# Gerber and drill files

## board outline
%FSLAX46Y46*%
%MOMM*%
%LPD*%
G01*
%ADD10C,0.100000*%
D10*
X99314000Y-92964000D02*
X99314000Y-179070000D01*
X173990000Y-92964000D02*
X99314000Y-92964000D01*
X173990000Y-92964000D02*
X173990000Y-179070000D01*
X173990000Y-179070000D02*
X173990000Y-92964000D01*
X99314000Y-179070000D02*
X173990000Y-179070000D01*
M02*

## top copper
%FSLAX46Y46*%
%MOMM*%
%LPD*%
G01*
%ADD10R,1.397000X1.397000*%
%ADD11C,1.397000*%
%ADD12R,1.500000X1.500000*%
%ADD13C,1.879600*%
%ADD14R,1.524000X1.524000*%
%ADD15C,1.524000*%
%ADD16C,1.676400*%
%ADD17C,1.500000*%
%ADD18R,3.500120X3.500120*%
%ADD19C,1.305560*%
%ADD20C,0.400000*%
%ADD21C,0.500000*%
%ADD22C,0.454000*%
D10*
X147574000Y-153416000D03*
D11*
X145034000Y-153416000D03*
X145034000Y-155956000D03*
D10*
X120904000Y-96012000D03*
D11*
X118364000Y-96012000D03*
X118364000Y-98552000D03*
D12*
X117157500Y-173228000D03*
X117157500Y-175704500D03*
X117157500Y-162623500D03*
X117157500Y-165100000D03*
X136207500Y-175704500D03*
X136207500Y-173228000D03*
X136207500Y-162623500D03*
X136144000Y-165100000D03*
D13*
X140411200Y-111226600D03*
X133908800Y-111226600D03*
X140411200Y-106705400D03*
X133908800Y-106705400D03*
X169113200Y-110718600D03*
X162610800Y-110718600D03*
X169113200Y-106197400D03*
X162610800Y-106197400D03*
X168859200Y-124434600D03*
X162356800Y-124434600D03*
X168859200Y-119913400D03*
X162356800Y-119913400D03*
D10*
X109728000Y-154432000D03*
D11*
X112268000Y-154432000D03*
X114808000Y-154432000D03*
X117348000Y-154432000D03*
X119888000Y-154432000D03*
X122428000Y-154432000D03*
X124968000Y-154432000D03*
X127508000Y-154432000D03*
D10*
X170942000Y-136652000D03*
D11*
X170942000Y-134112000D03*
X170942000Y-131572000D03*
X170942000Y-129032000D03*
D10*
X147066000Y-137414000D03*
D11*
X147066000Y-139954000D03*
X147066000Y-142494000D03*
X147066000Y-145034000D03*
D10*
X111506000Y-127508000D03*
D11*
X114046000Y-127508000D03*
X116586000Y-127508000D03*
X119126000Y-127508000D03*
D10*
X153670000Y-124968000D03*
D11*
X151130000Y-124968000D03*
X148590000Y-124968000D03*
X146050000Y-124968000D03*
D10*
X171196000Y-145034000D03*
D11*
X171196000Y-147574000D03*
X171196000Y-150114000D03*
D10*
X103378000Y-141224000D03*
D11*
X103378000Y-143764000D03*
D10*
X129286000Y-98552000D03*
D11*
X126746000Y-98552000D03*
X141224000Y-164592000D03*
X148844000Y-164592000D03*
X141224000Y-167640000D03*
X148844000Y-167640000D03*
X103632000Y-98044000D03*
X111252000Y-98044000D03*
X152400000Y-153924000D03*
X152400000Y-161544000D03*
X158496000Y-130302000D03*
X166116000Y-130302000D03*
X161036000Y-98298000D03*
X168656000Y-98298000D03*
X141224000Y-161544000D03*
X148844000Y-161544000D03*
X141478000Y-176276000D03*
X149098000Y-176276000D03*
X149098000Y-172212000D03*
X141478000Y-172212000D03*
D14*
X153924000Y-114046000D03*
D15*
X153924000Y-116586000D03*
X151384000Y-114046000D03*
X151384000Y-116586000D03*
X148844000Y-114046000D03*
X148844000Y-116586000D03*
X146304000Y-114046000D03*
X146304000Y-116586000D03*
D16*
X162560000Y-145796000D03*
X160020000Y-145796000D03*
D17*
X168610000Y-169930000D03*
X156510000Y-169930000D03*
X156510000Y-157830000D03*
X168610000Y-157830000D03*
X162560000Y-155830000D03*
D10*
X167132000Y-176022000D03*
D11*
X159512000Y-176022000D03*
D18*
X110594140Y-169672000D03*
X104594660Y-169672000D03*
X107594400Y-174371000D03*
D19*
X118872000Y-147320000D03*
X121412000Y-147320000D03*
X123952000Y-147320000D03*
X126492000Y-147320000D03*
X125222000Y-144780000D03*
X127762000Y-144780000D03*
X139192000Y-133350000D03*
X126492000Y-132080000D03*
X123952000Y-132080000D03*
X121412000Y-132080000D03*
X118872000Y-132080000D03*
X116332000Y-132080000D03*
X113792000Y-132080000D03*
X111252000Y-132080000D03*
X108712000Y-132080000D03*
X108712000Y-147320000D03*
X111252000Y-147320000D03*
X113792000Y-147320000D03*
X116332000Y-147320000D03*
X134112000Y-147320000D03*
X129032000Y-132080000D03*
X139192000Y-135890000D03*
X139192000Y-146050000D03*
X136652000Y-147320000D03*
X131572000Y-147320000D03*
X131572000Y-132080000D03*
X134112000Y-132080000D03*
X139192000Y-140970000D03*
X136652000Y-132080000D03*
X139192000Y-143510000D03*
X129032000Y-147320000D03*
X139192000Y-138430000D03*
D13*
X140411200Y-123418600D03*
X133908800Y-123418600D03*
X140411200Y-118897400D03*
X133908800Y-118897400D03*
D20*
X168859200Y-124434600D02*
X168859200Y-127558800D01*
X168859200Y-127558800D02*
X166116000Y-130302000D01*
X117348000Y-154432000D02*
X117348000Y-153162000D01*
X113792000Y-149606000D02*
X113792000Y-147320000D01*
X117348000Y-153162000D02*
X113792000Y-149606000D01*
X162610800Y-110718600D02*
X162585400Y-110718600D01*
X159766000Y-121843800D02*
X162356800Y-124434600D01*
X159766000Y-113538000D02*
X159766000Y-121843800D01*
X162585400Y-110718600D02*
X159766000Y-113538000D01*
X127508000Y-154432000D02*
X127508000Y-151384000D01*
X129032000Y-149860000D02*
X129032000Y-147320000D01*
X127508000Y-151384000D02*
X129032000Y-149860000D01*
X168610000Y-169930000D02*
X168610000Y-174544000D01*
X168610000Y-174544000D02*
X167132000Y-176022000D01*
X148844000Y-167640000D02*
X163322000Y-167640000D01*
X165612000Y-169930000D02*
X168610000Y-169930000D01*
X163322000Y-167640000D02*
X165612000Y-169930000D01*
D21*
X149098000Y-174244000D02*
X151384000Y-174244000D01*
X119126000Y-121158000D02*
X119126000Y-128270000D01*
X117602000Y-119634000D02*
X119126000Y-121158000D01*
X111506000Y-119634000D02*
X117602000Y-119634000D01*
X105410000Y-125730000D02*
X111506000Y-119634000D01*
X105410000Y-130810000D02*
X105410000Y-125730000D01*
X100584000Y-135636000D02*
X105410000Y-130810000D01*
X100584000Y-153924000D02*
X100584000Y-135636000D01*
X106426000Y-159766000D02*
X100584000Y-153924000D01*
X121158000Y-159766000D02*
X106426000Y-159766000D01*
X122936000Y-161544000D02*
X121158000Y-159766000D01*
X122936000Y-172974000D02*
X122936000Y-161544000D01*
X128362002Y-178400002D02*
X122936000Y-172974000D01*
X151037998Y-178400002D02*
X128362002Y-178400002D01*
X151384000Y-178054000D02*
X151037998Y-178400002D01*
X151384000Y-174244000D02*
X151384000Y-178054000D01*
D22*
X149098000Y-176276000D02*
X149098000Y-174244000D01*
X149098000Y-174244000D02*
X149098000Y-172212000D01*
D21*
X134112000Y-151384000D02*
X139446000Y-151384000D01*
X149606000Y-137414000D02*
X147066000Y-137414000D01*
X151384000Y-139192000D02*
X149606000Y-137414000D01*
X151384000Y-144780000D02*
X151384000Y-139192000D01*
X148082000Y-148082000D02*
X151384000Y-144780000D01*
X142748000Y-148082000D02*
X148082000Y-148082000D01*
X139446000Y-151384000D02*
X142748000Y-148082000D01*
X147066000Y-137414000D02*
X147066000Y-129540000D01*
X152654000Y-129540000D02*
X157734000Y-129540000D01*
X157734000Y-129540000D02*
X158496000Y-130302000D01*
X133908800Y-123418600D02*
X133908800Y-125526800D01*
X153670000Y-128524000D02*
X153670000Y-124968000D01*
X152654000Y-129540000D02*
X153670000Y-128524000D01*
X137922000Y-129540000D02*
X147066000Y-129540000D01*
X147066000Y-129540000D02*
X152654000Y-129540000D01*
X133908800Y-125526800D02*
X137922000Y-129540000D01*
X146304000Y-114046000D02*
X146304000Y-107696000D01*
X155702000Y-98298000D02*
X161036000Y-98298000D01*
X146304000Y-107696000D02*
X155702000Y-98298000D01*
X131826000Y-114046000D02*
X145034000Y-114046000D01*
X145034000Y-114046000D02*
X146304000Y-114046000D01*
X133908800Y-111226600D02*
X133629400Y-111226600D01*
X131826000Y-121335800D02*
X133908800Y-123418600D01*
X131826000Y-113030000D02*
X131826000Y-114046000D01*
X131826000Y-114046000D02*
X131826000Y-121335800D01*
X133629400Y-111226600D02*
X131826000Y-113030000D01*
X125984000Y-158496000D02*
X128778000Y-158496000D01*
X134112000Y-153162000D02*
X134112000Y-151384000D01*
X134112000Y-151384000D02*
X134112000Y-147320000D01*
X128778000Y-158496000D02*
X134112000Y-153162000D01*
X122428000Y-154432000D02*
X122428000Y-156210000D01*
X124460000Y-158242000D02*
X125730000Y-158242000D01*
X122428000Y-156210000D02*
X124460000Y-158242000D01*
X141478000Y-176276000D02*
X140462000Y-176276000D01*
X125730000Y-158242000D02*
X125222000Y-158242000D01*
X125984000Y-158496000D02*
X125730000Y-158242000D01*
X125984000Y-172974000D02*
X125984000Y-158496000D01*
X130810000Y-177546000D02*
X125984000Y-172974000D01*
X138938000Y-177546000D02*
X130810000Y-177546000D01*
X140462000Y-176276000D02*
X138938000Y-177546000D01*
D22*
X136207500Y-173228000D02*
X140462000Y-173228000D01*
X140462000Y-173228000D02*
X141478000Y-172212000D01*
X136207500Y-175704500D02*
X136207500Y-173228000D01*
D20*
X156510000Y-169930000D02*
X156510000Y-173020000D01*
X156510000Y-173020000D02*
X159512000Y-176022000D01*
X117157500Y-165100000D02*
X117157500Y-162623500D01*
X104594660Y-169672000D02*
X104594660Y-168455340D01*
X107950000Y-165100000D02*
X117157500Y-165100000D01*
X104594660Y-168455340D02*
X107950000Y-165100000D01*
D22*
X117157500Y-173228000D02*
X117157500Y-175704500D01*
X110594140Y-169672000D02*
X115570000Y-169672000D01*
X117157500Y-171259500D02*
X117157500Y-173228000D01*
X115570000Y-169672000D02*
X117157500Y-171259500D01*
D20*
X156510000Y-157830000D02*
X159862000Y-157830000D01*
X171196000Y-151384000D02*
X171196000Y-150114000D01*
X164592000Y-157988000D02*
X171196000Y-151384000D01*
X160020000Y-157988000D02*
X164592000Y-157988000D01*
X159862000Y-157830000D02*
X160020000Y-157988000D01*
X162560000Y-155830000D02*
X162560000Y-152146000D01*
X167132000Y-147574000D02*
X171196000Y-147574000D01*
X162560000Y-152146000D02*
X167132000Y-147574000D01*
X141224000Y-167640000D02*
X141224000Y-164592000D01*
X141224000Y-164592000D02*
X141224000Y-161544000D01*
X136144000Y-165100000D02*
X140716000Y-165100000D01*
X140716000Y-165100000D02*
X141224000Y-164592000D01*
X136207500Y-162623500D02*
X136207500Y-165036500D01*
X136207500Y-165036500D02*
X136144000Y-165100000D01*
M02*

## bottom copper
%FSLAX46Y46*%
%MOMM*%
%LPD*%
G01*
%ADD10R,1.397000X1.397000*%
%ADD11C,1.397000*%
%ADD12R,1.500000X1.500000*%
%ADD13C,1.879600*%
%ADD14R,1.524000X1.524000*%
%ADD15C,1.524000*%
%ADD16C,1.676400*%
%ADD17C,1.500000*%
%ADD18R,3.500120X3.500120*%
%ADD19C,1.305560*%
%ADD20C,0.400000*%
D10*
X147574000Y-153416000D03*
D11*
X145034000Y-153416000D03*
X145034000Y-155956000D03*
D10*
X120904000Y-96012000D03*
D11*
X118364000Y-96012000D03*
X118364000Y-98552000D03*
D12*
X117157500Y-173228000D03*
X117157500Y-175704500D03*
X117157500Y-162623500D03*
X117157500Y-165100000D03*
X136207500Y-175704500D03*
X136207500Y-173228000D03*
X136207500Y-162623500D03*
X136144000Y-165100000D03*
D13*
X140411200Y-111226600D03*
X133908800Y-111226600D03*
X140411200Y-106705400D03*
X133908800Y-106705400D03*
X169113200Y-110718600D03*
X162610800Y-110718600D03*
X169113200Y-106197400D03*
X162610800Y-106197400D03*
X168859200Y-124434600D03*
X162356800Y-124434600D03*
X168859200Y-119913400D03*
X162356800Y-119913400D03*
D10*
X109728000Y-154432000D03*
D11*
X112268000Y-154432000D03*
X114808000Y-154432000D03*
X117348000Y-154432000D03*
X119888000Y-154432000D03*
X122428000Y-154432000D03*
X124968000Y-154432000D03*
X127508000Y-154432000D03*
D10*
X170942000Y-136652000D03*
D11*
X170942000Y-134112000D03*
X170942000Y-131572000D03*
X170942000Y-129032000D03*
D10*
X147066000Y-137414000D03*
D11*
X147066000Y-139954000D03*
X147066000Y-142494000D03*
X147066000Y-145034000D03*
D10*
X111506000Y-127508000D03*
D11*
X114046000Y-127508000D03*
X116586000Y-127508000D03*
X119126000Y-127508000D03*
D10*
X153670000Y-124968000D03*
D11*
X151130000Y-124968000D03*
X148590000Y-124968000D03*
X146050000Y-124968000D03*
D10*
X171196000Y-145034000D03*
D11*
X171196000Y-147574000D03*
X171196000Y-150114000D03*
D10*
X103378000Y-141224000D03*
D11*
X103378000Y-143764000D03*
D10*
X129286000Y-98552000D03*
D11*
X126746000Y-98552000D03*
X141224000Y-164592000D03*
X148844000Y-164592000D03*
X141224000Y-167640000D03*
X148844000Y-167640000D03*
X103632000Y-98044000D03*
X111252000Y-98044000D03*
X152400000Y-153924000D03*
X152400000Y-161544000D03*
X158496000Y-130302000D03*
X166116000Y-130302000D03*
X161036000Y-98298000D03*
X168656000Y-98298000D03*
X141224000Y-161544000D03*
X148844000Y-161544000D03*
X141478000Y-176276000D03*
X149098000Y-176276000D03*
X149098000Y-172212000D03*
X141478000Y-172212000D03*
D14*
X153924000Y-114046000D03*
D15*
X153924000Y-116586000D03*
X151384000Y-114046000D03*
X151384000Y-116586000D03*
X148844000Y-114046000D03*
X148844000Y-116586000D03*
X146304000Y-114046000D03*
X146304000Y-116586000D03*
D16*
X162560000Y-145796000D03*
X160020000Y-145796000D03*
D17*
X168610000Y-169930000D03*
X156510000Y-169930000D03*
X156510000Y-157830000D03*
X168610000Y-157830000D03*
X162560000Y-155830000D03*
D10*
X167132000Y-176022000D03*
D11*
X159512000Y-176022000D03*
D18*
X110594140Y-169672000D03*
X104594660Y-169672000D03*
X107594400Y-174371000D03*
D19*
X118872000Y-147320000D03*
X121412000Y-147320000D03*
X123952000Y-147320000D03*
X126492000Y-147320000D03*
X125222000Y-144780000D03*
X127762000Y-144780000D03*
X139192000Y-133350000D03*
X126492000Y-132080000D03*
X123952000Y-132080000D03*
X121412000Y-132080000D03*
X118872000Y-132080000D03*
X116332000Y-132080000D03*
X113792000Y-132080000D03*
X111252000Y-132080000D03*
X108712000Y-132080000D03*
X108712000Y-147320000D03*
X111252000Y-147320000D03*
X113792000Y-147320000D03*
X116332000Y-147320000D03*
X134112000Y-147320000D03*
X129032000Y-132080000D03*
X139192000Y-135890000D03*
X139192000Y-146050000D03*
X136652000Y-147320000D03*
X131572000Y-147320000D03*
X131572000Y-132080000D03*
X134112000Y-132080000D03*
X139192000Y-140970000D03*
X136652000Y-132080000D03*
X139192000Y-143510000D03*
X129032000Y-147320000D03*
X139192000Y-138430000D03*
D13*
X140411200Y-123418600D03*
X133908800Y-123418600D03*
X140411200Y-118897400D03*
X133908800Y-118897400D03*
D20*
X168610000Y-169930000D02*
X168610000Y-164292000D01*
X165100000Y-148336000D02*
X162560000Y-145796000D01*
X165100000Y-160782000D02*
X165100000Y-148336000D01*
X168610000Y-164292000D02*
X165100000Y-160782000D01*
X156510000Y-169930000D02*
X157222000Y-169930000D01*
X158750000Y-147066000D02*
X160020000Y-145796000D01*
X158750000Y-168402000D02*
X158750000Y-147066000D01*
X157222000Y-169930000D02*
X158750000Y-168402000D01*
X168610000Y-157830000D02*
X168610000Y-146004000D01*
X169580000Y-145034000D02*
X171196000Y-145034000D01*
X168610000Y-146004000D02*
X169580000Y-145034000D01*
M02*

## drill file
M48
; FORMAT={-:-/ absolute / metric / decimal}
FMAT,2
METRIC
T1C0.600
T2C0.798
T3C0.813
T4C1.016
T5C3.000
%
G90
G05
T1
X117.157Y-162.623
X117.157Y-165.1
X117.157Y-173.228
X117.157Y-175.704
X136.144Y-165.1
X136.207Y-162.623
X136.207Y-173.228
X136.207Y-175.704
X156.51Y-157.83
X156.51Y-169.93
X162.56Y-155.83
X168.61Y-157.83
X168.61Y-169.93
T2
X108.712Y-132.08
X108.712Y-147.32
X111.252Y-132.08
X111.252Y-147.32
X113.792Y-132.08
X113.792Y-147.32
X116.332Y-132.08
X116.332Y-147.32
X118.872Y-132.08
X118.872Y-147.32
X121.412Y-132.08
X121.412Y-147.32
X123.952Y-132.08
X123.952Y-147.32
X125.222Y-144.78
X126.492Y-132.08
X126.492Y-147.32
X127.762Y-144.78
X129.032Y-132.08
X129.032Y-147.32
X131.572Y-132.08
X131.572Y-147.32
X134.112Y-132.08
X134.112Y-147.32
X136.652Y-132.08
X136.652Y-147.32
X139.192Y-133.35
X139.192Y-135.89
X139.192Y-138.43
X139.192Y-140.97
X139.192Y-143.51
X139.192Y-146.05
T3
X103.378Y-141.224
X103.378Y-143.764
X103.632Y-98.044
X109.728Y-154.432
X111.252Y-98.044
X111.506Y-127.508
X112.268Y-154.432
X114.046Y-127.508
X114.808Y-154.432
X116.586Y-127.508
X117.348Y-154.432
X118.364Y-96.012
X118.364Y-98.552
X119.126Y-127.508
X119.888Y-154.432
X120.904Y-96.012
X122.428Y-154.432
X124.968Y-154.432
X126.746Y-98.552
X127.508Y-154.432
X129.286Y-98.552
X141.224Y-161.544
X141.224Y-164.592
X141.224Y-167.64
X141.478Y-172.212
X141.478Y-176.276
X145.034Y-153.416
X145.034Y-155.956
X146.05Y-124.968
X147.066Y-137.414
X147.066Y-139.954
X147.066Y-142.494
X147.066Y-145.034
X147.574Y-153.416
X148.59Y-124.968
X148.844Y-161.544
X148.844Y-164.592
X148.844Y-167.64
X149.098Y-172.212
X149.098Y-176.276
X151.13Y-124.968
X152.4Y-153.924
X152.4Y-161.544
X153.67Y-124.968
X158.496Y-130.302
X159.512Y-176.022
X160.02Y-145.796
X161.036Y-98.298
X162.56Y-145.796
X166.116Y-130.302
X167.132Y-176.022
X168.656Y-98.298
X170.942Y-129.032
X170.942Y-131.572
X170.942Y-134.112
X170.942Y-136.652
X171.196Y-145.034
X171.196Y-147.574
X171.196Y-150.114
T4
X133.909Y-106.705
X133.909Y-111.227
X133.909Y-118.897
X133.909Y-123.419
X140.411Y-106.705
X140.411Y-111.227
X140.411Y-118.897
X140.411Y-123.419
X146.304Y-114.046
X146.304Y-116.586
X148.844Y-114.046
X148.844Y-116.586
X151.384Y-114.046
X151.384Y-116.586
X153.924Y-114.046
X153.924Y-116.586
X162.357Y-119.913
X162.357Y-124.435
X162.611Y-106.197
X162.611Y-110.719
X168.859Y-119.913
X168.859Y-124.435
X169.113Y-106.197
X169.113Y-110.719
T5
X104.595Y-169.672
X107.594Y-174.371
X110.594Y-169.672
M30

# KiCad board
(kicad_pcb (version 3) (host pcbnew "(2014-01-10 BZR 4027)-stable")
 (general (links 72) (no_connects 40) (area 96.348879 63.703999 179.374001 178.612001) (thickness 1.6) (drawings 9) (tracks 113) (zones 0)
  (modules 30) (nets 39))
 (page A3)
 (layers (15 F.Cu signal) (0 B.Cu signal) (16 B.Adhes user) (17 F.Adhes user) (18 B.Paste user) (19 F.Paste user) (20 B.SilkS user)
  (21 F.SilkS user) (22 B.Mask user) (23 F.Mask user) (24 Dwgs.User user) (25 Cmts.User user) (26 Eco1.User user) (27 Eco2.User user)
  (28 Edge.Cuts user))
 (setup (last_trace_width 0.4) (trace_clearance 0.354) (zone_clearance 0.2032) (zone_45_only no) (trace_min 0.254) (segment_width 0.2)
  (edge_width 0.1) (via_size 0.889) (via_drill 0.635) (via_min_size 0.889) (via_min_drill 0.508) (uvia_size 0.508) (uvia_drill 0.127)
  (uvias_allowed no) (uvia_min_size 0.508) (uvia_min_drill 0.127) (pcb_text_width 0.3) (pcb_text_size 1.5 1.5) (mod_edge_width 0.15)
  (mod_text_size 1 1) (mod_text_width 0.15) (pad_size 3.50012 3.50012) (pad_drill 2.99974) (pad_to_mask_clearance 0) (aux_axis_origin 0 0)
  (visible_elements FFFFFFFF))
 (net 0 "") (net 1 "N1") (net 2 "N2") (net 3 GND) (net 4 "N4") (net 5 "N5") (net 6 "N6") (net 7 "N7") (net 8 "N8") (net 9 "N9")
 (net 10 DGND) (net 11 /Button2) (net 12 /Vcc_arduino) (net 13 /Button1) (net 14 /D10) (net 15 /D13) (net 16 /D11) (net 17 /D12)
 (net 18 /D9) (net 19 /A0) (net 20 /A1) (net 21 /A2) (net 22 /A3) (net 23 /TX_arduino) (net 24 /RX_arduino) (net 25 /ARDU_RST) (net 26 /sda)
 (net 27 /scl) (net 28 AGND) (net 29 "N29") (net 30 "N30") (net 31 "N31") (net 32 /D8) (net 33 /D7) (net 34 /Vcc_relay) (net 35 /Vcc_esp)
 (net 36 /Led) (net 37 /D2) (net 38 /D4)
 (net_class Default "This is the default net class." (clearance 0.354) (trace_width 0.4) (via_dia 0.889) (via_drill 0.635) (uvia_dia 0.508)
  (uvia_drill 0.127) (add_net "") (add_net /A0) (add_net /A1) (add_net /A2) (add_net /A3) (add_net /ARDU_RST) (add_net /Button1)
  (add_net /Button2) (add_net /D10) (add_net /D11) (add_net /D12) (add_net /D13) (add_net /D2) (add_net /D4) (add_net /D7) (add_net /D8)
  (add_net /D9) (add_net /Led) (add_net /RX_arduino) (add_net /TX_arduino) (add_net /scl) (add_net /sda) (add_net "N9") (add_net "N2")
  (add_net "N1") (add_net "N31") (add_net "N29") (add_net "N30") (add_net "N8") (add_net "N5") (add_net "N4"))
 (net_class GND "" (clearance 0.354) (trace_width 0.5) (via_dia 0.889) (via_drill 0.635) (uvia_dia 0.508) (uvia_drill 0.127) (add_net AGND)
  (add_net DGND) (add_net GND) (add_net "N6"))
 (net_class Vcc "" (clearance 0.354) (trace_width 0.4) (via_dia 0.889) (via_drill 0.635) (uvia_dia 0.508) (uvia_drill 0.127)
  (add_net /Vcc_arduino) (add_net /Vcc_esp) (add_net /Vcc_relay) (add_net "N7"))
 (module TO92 (layer F.Cu) (at 146.304 154.686)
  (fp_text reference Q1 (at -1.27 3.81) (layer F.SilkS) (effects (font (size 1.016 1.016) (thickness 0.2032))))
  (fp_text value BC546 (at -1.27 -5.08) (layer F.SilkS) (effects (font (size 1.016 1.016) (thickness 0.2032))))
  (pad 1 thru_hole rect (at 1.27 -1.27) (size 1.397 1.397) (drill 0.8128) (layers *.Cu *.Mask F.SilkS) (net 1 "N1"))
  (pad 2 thru_hole circle (at -1.27 -1.27) (size 1.397 1.397) (drill 0.8128) (layers *.Cu *.Mask F.SilkS) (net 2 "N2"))
  (pad 3 thru_hole circle (at -1.27 1.27) (size 1.397 1.397) (drill 0.8128) (layers *.Cu *.Mask F.SilkS) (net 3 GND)))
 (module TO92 (layer F.Cu) (at 119.634 97.282)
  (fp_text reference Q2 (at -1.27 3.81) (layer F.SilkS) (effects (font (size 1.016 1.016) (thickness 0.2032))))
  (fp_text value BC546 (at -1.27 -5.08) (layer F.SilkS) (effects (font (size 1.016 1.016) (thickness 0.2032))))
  (pad 1 thru_hole rect (at 1.27 -1.27) (size 1.397 1.397) (drill 0.8128) (layers *.Cu *.Mask F.SilkS) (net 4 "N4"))
  (pad 2 thru_hole circle (at -1.27 -1.27) (size 1.397 1.397) (drill 0.8128) (layers *.Cu *.Mask F.SilkS) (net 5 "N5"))
  (pad 3 thru_hole circle (at -1.27 1.27) (size 1.397 1.397) (drill 0.8128) (layers *.Cu *.Mask F.SilkS) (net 3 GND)))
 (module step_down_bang (layer F.Cu) (at 126.492 169.164 90)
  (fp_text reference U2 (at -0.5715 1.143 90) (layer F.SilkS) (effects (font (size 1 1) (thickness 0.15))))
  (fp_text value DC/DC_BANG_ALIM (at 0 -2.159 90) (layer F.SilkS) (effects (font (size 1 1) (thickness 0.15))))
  (pad 3 thru_hole rect (at -4.064 -9.3345 90) (size 1.5 1.5) (drill 0.6) (layers *.Cu *.Mask F.SilkS) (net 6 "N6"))
  (pad 4 thru_hole rect (at -6.5405 -9.3345 90) (size 1.5 1.5) (drill 0.6) (layers *.Cu *.Mask F.SilkS) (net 6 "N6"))
  (pad 1 thru_hole rect (at 6.5405 -9.3345 90) (size 1.5 1.5) (drill 0.6) (layers *.Cu *.Mask F.SilkS) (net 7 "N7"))
  (pad 2 thru_hole rect (at 4.064 -9.3345 90) (size 1.5 1.5) (drill 0.6) (layers *.Cu *.Mask F.SilkS) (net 7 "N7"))
  (pad 8 thru_hole rect (at -6.5405 9.7155 90) (size 1.5 1.5) (drill 0.6) (layers *.Cu *.Mask F.SilkS) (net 3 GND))
  (pad 7 thru_hole rect (at -4.064 9.7155 90) (size 1.5 1.5) (drill 0.6) (layers *.Cu *.Mask F.SilkS) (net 3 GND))
  (pad 5 thru_hole rect (at 6.5405 9.7155 90) (size 1.5 1.5) (drill 0.6) (layers *.Cu *.Mask F.SilkS) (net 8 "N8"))
  (pad 6 thru_hole rect (at 4.064 9.652 90) (size 1.5 1.5) (drill 0.6) (layers *.Cu *.Mask F.SilkS) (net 8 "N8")))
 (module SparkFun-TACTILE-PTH (layer F.Cu) (at 137.16 108.966 180)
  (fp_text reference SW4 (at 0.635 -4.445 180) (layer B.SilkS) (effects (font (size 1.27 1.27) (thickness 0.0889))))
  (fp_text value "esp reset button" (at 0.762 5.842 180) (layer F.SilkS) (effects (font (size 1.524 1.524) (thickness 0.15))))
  (pad 1 thru_hole circle (at -3.2512 -2.2606 180) (size 1.8796 1.8796) (drill 1.016) (layers *.Cu F.Paste F.SilkS F.Mask) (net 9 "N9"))
  (pad 2 thru_hole circle (at 3.2512 -2.2606 180) (size 1.8796 1.8796) (drill 1.016) (layers *.Cu F.Paste F.SilkS F.Mask) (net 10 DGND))
  (pad 3 thru_hole circle (at -3.2512 2.2606 180) (size 1.8796 1.8796) (drill 1.016) (layers *.Cu F.Paste F.SilkS F.Mask))
  (pad 4 thru_hole circle (at 3.2512 2.2606 180) (size 1.8796 1.8796) (drill 1.016) (layers *.Cu F.Paste F.SilkS F.Mask)))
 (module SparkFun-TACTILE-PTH (layer F.Cu) (at 165.862 108.458 180)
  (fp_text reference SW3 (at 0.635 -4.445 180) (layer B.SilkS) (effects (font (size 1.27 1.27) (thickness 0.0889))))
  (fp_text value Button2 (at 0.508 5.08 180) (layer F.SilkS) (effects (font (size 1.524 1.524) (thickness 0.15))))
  (pad 1 thru_hole circle (at -3.2512 -2.2606 180) (size 1.8796 1.8796) (drill 1.016) (layers *.Cu F.Paste F.SilkS F.Mask) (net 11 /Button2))
  (pad 2 thru_hole circle (at 3.2512 -2.2606 180) (size 1.8796 1.8796) (drill 1.016) (layers *.Cu F.Paste F.SilkS F.Mask)
   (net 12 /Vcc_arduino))
  (pad 3 thru_hole circle (at -3.2512 2.2606 180) (size 1.8796 1.8796) (drill 1.016) (layers *.Cu F.Paste F.SilkS F.Mask))
  (pad 4 thru_hole circle (at 3.2512 2.2606 180) (size 1.8796 1.8796) (drill 1.016) (layers *.Cu F.Paste F.SilkS F.Mask)))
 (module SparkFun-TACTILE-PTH (layer F.Cu) (at 165.608 122.174 180)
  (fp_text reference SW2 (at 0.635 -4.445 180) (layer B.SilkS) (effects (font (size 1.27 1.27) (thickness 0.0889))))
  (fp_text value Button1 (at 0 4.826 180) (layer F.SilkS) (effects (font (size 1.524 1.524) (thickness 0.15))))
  (pad 1 thru_hole circle (at -3.2512 -2.2606 180) (size 1.8796 1.8796) (drill 1.016) (layers *.Cu F.Paste F.SilkS F.Mask) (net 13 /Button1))
  (pad 2 thru_hole circle (at 3.2512 -2.2606 180) (size 1.8796 1.8796) (drill 1.016) (layers *.Cu F.Paste F.SilkS F.Mask)
   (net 12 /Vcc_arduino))
  (pad 3 thru_hole circle (at -3.2512 2.2606 180) (size 1.8796 1.8796) (drill 1.016) (layers *.Cu F.Paste F.SilkS F.Mask))
  (pad 4 thru_hole circle (at 3.2512 2.2606 180) (size 1.8796 1.8796) (drill 1.016) (layers *.Cu F.Paste F.SilkS F.Mask)))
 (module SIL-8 (layer F.Cu) (at 118.618 154.432)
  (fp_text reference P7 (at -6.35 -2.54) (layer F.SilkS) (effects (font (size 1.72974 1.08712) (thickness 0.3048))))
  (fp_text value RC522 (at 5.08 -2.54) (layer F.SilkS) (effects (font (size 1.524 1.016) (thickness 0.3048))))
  (pad 1 thru_hole rect (at -8.89 0) (size 1.397 1.397) (drill 0.8128) (layers *.Cu *.Mask F.SilkS) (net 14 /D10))
  (pad 2 thru_hole circle (at -6.35 0) (size 1.397 1.397) (drill 0.8128) (layers *.Cu *.Mask F.SilkS) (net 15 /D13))
  (pad 3 thru_hole circle (at -3.81 0) (size 1.397 1.397) (drill 0.8128) (layers *.Cu *.Mask F.SilkS) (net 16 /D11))
  (pad 4 thru_hole circle (at -1.27 0) (size 1.397 1.397) (drill 0.8128) (layers *.Cu *.Mask F.SilkS) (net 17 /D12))
  (pad 5 thru_hole circle (at 1.27 0) (size 1.397 1.397) (drill 0.8128) (layers *.Cu *.Mask F.SilkS))
  (pad 6 thru_hole circle (at 3.81 0) (size 1.397 1.397) (drill 0.8128) (layers *.Cu *.Mask F.SilkS) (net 10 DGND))
  (pad 7 thru_hole circle (at 6.35 0) (size 1.397 1.397) (drill 0.8128) (layers *.Cu *.Mask F.SilkS) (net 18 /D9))
  (pad 8 thru_hole circle (at 8.89 0) (size 1.397 1.397) (drill 0.8128) (layers *.Cu *.Mask F.SilkS) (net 12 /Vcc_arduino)))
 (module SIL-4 (layer F.Cu) (at 170.942 132.842 90)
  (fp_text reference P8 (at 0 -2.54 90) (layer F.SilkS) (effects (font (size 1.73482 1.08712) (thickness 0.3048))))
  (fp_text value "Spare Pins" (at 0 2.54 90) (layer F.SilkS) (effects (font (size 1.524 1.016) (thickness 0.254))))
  (pad 1 thru_hole rect (at -3.81 0 90) (size 1.397 1.397) (drill 0.8128) (layers *.Cu *.Mask F.SilkS) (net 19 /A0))
  (pad 2 thru_hole circle (at -1.27 0 90) (size 1.397 1.397) (drill 0.8128) (layers *.Cu *.Mask F.SilkS) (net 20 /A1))
  (pad 3 thru_hole circle (at 1.27 0 90) (size 1.397 1.397) (drill 0.8128) (layers *.Cu *.Mask F.SilkS) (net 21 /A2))
  (pad 4 thru_hole circle (at 3.81 0 90) (size 1.397 1.397) (drill 0.8128) (layers *.Cu *.Mask F.SilkS) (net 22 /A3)))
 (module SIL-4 (layer F.Cu) (at 147.066 141.224 270)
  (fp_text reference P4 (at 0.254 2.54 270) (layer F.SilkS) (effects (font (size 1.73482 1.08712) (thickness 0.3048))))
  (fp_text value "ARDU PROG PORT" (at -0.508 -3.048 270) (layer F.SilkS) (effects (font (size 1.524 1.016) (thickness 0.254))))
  (pad 1 thru_hole rect (at -3.81 0 270) (size 1.397 1.397) (drill 0.8128) (layers *.Cu *.Mask F.SilkS) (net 10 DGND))
  (pad 2 thru_hole circle (at -1.27 0 270) (size 1.397 1.397) (drill 0.8128) (layers *.Cu *.Mask F.SilkS) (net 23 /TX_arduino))
  (pad 3 thru_hole circle (at 1.27 0 270) (size 1.397 1.397) (drill 0.8128) (layers *.Cu *.Mask F.SilkS) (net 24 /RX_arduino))
  (pad 4 thru_hole circle (at 3.81 0 270) (size 1.397 1.397) (drill 0.8128) (layers *.Cu *.Mask F.SilkS) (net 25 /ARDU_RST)))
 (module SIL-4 (layer F.Cu) (at 115.316 127.508)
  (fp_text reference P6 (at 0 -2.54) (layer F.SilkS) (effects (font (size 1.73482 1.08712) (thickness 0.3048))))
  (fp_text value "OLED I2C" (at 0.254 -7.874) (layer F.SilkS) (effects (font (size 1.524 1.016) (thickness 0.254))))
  (pad 1 thru_hole rect (at -3.81 0) (size 1.397 1.397) (drill 0.8128) (layers *.Cu *.Mask F.SilkS) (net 12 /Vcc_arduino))
  (pad 2 thru_hole circle (at -1.27 0) (size 1.397 1.397) (drill 0.8128) (layers *.Cu *.Mask F.SilkS) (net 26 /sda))
  (pad 3 thru_hole circle (at 1.27 0) (size 1.397 1.397) (drill 0.8128) (layers *.Cu *.Mask F.SilkS) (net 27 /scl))
  (pad 4 thru_hole circle (at 3.81 0) (size 1.397 1.397) (drill 0.8128) (layers *.Cu *.Mask F.SilkS) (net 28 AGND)))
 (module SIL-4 (layer F.Cu) (at 149.86 124.968 180)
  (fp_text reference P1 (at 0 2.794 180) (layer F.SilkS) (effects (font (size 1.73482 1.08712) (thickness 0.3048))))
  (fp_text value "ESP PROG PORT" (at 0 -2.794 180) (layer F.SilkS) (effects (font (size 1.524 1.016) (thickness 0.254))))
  (pad 1 thru_hole rect (at -3.81 0 180) (size 1.397 1.397) (drill 0.8128) (layers *.Cu *.Mask F.SilkS) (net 10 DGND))
  (pad 2 thru_hole circle (at -1.27 0 180) (size 1.397 1.397) (drill 0.8128) (layers *.Cu *.Mask F.SilkS) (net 24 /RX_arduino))
  (pad 3 thru_hole circle (at 1.27 0 180) (size 1.397 1.397) (drill 0.8128) (layers *.Cu *.Mask F.SilkS) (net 23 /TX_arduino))
  (pad 4 thru_hole circle (at 3.81 0 180) (size 1.397 1.397) (drill 0.8128) (layers *.Cu *.Mask F.SilkS)))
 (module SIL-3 (layer F.Cu) (at 171.196 147.574 270)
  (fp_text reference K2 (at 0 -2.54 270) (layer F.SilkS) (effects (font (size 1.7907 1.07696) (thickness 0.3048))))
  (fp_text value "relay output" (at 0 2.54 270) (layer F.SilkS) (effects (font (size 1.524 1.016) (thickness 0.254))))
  (pad 1 thru_hole rect (at -2.54 0 270) (size 1.397 1.397) (drill 0.8128) (layers *.Cu *.Mask F.SilkS) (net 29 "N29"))
  (pad 2 thru_hole circle (at 0 0 270) (size 1.397 1.397) (drill 0.8128) (layers *.Cu *.Mask F.SilkS) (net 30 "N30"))
  (pad 3 thru_hole circle (at 2.54 0 270) (size 1.397 1.397) (drill 0.8128) (layers *.Cu *.Mask F.SilkS) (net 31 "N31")))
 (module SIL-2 (layer F.Cu) (at 103.378 142.494 270)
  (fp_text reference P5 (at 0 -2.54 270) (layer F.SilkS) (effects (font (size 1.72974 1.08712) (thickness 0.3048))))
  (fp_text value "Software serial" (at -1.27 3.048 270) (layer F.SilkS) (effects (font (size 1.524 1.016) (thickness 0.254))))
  (pad 1 thru_hole rect (at -1.27 0 270) (size 1.397 1.397) (drill 0.8128) (layers *.Cu *.Mask F.SilkS) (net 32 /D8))
  (pad 2 thru_hole circle (at 1.27 0 270) (size 1.397 1.397) (drill 0.8128) (layers *.Cu *.Mask F.SilkS) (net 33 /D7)))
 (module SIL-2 (layer F.Cu) (at 128.016 98.552 180)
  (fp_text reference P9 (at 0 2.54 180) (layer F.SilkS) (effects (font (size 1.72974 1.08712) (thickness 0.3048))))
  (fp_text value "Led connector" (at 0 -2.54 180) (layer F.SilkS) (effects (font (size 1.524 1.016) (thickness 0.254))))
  (pad 1 thru_hole rect (at -1.27 0 180) (size 1.397 1.397) (drill 0.8128) (layers *.Cu *.Mask F.SilkS) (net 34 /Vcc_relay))
  (pad 2 thru_hole circle (at 1.27 0 180) (size 1.397 1.397) (drill 0.8128) (layers *.Cu *.Mask F.SilkS) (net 4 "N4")))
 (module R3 (layer F.Cu) (at 145.034 164.592) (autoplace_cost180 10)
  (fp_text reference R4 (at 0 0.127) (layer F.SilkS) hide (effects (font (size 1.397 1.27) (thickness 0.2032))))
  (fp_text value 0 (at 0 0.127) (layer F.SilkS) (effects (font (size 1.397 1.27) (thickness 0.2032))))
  (pad 1 thru_hole circle (at -3.81 0) (size 1.397 1.397) (drill 0.8128) (layers *.Cu *.Mask F.SilkS) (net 8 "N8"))
  (pad 2 thru_hole circle (at 3.81 0) (size 1.397 1.397) (drill 0.8128) (layers *.Cu *.Mask F.SilkS) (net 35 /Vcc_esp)))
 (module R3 (layer F.Cu) (at 145.034 167.64) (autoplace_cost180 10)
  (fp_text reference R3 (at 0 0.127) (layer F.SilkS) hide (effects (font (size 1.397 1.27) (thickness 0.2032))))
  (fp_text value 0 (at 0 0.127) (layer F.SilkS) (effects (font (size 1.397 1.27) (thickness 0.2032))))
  (pad 1 thru_hole circle (at -3.81 0) (size 1.397 1.397) (drill 0.8128) (layers *.Cu *.Mask F.SilkS) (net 8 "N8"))
  (pad 2 thru_hole circle (at 3.81 0) (size 1.397 1.397) (drill 0.8128) (layers *.Cu *.Mask F.SilkS) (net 34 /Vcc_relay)))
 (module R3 (layer F.Cu) (at 107.442 98.044) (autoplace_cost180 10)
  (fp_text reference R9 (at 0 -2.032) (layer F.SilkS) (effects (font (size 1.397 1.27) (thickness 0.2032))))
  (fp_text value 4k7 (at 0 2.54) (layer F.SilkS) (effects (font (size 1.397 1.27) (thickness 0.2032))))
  (pad 1 thru_hole circle (at -3.81 0) (size 1.397 1.397) (drill 0.8128) (layers *.Cu *.Mask F.SilkS) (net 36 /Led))
  (pad 2 thru_hole circle (at 3.81 0) (size 1.397 1.397) (drill 0.8128) (layers *.Cu *.Mask F.SilkS) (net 5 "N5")))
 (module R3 (layer F.Cu) (at 152.4 157.734 270) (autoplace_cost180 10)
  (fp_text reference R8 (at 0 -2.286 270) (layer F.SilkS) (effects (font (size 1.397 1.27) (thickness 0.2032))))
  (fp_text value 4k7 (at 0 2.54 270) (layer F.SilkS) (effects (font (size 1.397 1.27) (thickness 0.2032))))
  (pad 1 thru_hole circle (at -3.81 0 270) (size 1.397 1.397) (drill 0.8128) (layers *.Cu *.Mask F.SilkS) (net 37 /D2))
  (pad 2 thru_hole circle (at 3.81 0 270) (size 1.397 1.397) (drill 0.8128) (layers *.Cu *.Mask F.SilkS) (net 2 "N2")))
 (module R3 (layer F.Cu) (at 162.306 130.302) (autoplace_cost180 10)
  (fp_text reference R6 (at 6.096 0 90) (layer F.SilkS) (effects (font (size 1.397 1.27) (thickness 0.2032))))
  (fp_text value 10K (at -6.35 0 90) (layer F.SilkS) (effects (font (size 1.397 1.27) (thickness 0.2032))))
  (pad 1 thru_hole circle (at -3.81 0) (size 1.397 1.397) (drill 0.8128) (layers *.Cu *.Mask F.SilkS) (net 10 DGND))
  (pad 2 thru_hole circle (at 3.81 0) (size 1.397 1.397) (drill 0.8128) (layers *.Cu *.Mask F.SilkS) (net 13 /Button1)))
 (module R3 (layer F.Cu) (at 164.846 98.298) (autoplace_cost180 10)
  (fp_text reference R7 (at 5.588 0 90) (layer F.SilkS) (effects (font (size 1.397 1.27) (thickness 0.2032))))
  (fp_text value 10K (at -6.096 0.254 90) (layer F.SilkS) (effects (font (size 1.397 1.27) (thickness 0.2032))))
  (pad 1 thru_hole circle (at -3.81 0) (size 1.397 1.397) (drill 0.8128) (layers *.Cu *.Mask F.SilkS) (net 10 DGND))
  (pad 2 thru_hole circle (at 3.81 0) (size 1.397 1.397) (drill 0.8128) (layers *.Cu *.Mask F.SilkS) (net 11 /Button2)))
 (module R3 (layer F.Cu) (at 145.034 161.544) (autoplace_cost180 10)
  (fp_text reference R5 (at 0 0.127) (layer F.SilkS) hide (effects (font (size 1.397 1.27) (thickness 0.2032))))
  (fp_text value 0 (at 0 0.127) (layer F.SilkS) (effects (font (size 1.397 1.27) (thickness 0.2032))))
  (pad 1 thru_hole circle (at -3.81 0) (size 1.397 1.397) (drill 0.8128) (layers *.Cu *.Mask F.SilkS) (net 8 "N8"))
  (pad 2 thru_hole circle (at 3.81 0) (size 1.397 1.397) (drill 0.8128) (layers *.Cu *.Mask F.SilkS) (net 12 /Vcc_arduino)))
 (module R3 (layer F.Cu) (at 145.288 176.276) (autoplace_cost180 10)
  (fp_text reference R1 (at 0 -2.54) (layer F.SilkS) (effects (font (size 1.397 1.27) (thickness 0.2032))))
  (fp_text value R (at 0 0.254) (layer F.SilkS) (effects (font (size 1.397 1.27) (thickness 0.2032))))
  (pad 1 thru_hole circle (at -3.81 0) (size 1.397 1.397) (drill 0.8128) (layers *.Cu *.Mask F.SilkS) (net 10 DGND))
  (pad 2 thru_hole circle (at 3.81 0) (size 1.397 1.397) (drill 0.8128) (layers *.Cu *.Mask F.SilkS) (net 28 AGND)))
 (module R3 (layer F.Cu) (at 145.288 172.212 180) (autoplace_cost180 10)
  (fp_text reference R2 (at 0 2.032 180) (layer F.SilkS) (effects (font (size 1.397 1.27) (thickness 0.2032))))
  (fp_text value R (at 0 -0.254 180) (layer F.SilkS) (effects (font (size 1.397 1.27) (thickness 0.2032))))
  (pad 1 thru_hole circle (at -3.81 0 180) (size 1.397 1.397) (drill 0.8128) (layers *.Cu *.Mask F.SilkS) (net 28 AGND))
  (pad 2 thru_hole circle (at 3.81 0 180) (size 1.397 1.397) (drill 0.8128) (layers *.Cu *.Mask F.SilkS) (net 3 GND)))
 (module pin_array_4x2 (layer F.Cu) (at 150.114 115.316 180)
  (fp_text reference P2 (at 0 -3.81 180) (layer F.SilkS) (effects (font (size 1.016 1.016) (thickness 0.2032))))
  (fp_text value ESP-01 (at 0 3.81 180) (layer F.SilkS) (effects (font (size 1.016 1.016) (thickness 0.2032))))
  (pad 1 thru_hole rect (at -3.81 1.27 180) (size 1.524 1.524) (drill 1.016) (layers *.Cu *.Mask F.SilkS) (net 24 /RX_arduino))
  (pad 2 thru_hole circle (at -3.81 -1.27 180) (size 1.524 1.524) (drill 1.016) (layers *.Cu *.Mask F.SilkS) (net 35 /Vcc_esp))
  (pad 3 thru_hole circle (at -1.27 1.27 180) (size 1.524 1.524) (drill 1.016) (layers *.Cu *.Mask F.SilkS) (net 25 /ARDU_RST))
  (pad 4 thru_hole circle (at -1.27 -1.27 180) (size 1.524 1.524) (drill 1.016) (layers *.Cu *.Mask F.SilkS) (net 9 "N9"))
  (pad 5 thru_hole circle (at 1.27 1.27 180) (size 1.524 1.524) (drill 1.016) (layers *.Cu *.Mask F.SilkS))
  (pad 6 thru_hole circle (at 1.27 -1.27 180) (size 1.524 1.524) (drill 1.016) (layers *.Cu *.Mask F.SilkS) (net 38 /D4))
  (pad 7 thru_hole circle (at 3.81 1.27 180) (size 1.524 1.524) (drill 1.016) (layers *.Cu *.Mask F.SilkS) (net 10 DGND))
  (pad 8 thru_hole circle (at 3.81 -1.27 180) (size 1.524 1.524) (drill 1.016) (layers *.Cu *.Mask F.SilkS) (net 23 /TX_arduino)))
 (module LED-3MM (layer F.Cu) (at 161.29 145.796 180)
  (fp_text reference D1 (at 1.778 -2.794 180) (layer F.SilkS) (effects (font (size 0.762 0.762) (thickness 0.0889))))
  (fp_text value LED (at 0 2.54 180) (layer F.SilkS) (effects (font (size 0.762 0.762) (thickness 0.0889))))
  (pad 1 thru_hole circle (at -1.27 0 180) (size 1.6764 1.6764) (drill 0.8128) (layers *.Cu *.Mask F.SilkS) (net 34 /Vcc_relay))
  (pad 2 thru_hole circle (at 1.27 0 180) (size 1.6764 1.6764) (drill 0.8128) (layers *.Cu *.Mask F.SilkS) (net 1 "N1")))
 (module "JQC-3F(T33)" (layer F.Cu) (at 162.56 163.83 270)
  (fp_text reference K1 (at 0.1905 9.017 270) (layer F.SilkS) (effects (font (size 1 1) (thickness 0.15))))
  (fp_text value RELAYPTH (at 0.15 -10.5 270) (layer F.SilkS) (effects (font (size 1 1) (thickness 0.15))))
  (pad 3 thru_hole circle (at 6.1 -6.05 270) (size 1.5 1.5) (drill 0.6) (layers *.Cu *.Mask F.SilkS) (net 34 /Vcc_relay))
  (pad 5 thru_hole circle (at 6.1 6.05 270) (size 1.5 1.5) (drill 0.6) (layers *.Cu *.Mask F.SilkS) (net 1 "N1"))
  (pad 2 thru_hole circle (at -6 6.05 270) (size 1.5 1.5) (drill 0.6) (layers *.Cu *.Mask F.SilkS) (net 31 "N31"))
  (pad 1 thru_hole circle (at -6 -6.05 270) (size 1.5 1.5) (drill 0.6) (layers *.Cu *.Mask F.SilkS) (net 29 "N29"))
  (pad 4 thru_hole circle (at -8 0 270) (size 1.5 1.5) (drill 0.6) (layers *.Cu *.Mask F.SilkS) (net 30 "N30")))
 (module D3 (layer F.Cu) (at 163.322 176.022)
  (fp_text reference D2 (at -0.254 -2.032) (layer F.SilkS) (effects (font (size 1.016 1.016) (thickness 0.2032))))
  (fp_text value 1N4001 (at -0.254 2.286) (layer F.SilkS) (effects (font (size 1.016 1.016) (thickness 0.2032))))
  (pad 2 thru_hole rect (at 3.81 0) (size 1.397 1.397) (drill 0.8128) (layers *.Cu *.Mask F.SilkS) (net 34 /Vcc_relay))
  (pad 1 thru_hole circle (at -3.81 0) (size 1.397 1.397) (drill 0.8128) (layers *.Cu *.Mask F.SilkS) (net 1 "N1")))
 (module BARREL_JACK (layer F.Cu) (at 104.394 169.672)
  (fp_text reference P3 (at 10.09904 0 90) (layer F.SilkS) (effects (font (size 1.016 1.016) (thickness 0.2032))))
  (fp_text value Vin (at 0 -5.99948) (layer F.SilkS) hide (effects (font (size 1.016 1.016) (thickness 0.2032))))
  (pad 1 thru_hole rect (at 6.20014 0) (size 3.50012 3.50012) (drill 2.99974) (layers *.Cu *.Mask F.SilkS) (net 6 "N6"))
  (pad 2 thru_hole rect (at 0.20066 0) (size 3.50012 3.50012) (drill 2.99974) (layers *.Cu *.Mask F.SilkS) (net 7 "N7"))
  (pad 3 thru_hole rect (at 3.2004 4.699) (size 3.50012 3.50012) (drill 2.99974) (layers *.Cu *.Mask F.SilkS)))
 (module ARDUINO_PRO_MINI (layer F.Cu) (at 125.222 139.7)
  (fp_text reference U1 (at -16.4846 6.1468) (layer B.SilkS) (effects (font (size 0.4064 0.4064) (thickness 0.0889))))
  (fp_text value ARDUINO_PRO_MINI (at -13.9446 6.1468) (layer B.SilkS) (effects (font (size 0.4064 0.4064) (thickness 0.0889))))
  (pad A0 thru_hole circle (at -6.35 7.62) (size 1.30556 1.30556) (drill 0.79756) (layers *.Cu F.Paste F.SilkS F.Mask) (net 19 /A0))
  (pad A1 thru_hole circle (at -3.81 7.62) (size 1.30556 1.30556) (drill 0.79756) (layers *.Cu F.Paste F.SilkS F.Mask) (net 20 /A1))
  (pad A2 thru_hole circle (at -1.27 7.62) (size 1.30556 1.30556) (drill 0.79756) (layers *.Cu F.Paste F.SilkS F.Mask) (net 21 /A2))
  (pad A3 thru_hole circle (at 1.27 7.62) (size 1.30556 1.30556) (drill 0.79756) (layers *.Cu F.Paste F.SilkS F.Mask) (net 22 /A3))
  (pad A4 thru_hole circle (at 0 5.08) (size 1.30556 1.30556) (drill 0.79756) (layers *.Cu F.Paste F.SilkS F.Mask) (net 26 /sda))
  (pad A5 thru_hole circle (at 2.54 5.08) (size 1.30556 1.30556) (drill 0.79756) (layers *.Cu F.Paste F.SilkS F.Mask) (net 27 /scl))
  (pad BLK thru_hole circle (at 13.97 -6.35) (size 1.30556 1.30556) (drill 0.79756) (layers *.Cu F.Paste F.SilkS F.Mask))
  (pad D2 thru_hole circle (at 1.27 -7.62) (size 1.30556 1.30556) (drill 0.79756) (layers *.Cu F.Paste F.SilkS F.Mask) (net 37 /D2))
  (pad D3 thru_hole circle (at -1.27 -7.62) (size 1.30556 1.30556) (drill 0.79756) (layers *.Cu F.Paste F.SilkS F.Mask) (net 11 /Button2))
  (pad D4 thru_hole circle (at -3.81 -7.62) (size 1.30556 1.30556) (drill 0.79756) (layers *.Cu F.Paste F.SilkS F.Mask) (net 38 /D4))
  (pad D5 thru_hole circle (at -6.35 -7.62) (size 1.30556 1.30556) (drill 0.79756) (layers *.Cu F.Paste F.SilkS F.Mask) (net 13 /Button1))
  (pad D6 thru_hole circle (at -8.89 -7.62) (size 1.30556 1.30556) (drill 0.79756) (layers *.Cu F.Paste F.SilkS F.Mask) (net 36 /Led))
  (pad D7 thru_hole circle (at -11.43 -7.62) (size 1.30556 1.30556) (drill 0.79756) (layers *.Cu F.Paste F.SilkS F.Mask) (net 33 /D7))
  (pad D8 thru_hole circle (at -13.97 -7.62) (size 1.30556 1.30556) (drill 0.79756) (layers *.Cu F.Paste F.SilkS F.Mask) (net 32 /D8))
  (pad D9 thru_hole circle (at -16.51 -7.62) (size 1.30556 1.30556) (drill 0.79756) (layers *.Cu F.Paste F.SilkS F.Mask) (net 18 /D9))
  (pad D10 thru_hole circle (at -16.51 7.62) (size 1.30556 1.30556) (drill 0.79756) (layers *.Cu F.Paste F.SilkS F.Mask) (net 14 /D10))
  (pad D11 thru_hole circle (at -13.97 7.62) (size 1.30556 1.30556) (drill 0.79756) (layers *.Cu F.Paste F.SilkS F.Mask) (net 16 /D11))
  (pad D12 thru_hole circle (at -11.43 7.62) (size 1.30556 1.30556) (drill 0.79756) (layers *.Cu F.Paste F.SilkS F.Mask) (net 17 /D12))
  (pad D13 thru_hole circle (at -8.89 7.62) (size 1.30556 1.30556) (drill 0.79756) (layers *.Cu F.Paste F.SilkS F.Mask) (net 15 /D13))
  (pad GND1 thru_hole circle (at 8.89 7.62) (size 1.30556 1.30556) (drill 0.79756) (layers *.Cu F.Paste F.SilkS F.Mask) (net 10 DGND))
  (pad GND2 thru_hole circle (at 3.81 -7.62) (size 1.30556 1.30556) (drill 0.79756) (layers *.Cu F.Paste F.SilkS F.Mask))
  (pad GND3 thru_hole circle (at 13.97 -3.81) (size 1.30556 1.30556) (drill 0.79756) (layers *.Cu F.Paste F.SilkS F.Mask))
  (pad GRN thru_hole circle (at 13.97 6.35) (size 1.30556 1.30556) (drill 0.79756) (layers *.Cu F.Paste F.SilkS F.Mask))
  (pad RAW thru_hole circle (at 11.43 7.62) (size 1.30556 1.30556) (drill 0.79756) (layers *.Cu F.Paste F.SilkS F.Mask))
  (pad RST1 thru_hole circle (at 6.35 7.62) (size 1.30556 1.30556) (drill 0.79756) (layers *.Cu F.Paste F.SilkS F.Mask) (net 25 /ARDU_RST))
  (pad RST2 thru_hole circle (at 6.35 -7.62) (size 1.30556 1.30556) (drill 0.79756) (layers *.Cu F.Paste F.SilkS F.Mask))
  (pad RXI thru_hole circle (at 8.89 -7.62) (size 1.30556 1.30556) (drill 0.79756) (layers *.Cu F.Paste F.SilkS F.Mask) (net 24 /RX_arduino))
  (pad RXI2 thru_hole circle (at 13.97 1.27) (size 1.30556 1.30556) (drill 0.79756) (layers *.Cu F.Paste F.SilkS F.Mask))
  (pad TXO thru_hole circle (at 11.43 -7.62) (size 1.30556 1.30556) (drill 0.79756) (layers *.Cu F.Paste F.SilkS F.Mask)
   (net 23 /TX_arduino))
  (pad TXO2 thru_hole circle (at 13.97 3.81) (size 1.30556 1.30556) (drill 0.79756) (layers *.Cu F.Paste F.SilkS F.Mask))
  (pad VCC1 thru_hole circle (at 3.81 7.62) (size 1.30556 1.30556) (drill 0.79756) (layers *.Cu F.Paste F.SilkS F.Mask)
   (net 12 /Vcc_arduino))
  (pad VCC2 thru_hole circle (at 13.97 -1.27) (size 1.30556 1.30556) (drill 0.79756) (layers *.Cu F.Paste F.SilkS F.Mask)))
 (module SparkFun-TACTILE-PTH (layer F.Cu) (at 137.16 121.158 180)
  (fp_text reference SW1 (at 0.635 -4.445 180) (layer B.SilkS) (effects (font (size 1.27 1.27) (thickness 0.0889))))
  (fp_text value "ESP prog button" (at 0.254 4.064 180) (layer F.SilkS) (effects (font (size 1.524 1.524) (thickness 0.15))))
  (pad 1 thru_hole circle (at -3.2512 -2.2606 180) (size 1.8796 1.8796) (drill 1.016) (layers *.Cu F.Paste F.SilkS F.Mask)
   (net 25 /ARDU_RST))
  (pad 2 thru_hole circle (at 3.2512 -2.2606 180) (size 1.8796 1.8796) (drill 1.016) (layers *.Cu F.Paste F.SilkS F.Mask) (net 10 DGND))
  (pad 3 thru_hole circle (at -3.2512 2.2606 180) (size 1.8796 1.8796) (drill 1.016) (layers *.Cu F.Paste F.SilkS F.Mask))
  (pad 4 thru_hole circle (at 3.2512 2.2606 180) (size 1.8796 1.8796) (drill 1.016) (layers *.Cu F.Paste F.SilkS F.Mask)))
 (gr_line (start 99.314 92.964) (end 99.314 179.07) (angle 90) (layer Edge.Cuts) (width 0.1))
 (gr_line (start 173.99 92.964) (end 99.314 92.964) (angle 90) (layer Edge.Cuts) (width 0.1))
 (gr_line (start 173.99 92.964) (end 173.99 179.07) (angle 90) (layer Edge.Cuts) (width 0.1))
 (gr_line (start 173.99 179.07) (end 173.99 92.964) (angle 90) (layer Edge.Cuts) (width 0.1))
 (gr_line (start 99.314 179.07) (end 173.99 179.07) (angle 90) (layer Edge.Cuts) (width 0.1))
 (segment (start 168.8592 124.4346) (end 168.8592 127.5588) (width 0.4) (layer F.Cu) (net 13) (status 400000))
 (segment (start 168.8592 127.5588) (end 166.116 130.302) (width 0.4) (layer F.Cu) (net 13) (status 800000))
 (segment (start 117.348 154.432) (end 117.348 153.162) (width 0.4) (layer F.Cu) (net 17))
 (segment (start 113.792 149.606) (end 113.792 147.32) (width 0.4) (layer F.Cu) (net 17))
 (segment (start 117.348 153.162) (end 113.792 149.606) (width 0.4) (layer F.Cu) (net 17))
 (segment (start 162.6108 110.7186) (end 162.5854 110.7186) (width 0.4) (layer F.Cu) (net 12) (status C00000))
 (segment (start 159.766 121.8438) (end 162.3568 124.4346) (width 0.4) (layer F.Cu) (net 12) (status 800000))
 (segment (start 159.766 113.538) (end 159.766 121.8438) (width 0.4) (layer F.Cu) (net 12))
 (segment (start 162.5854 110.7186) (end 159.766 113.538) (width 0.4) (layer F.Cu) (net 12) (status 400000))
 (segment (start 127.508 154.432) (end 127.508 151.384) (width 0.4) (layer F.Cu) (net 12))
 (segment (start 129.032 149.86) (end 129.032 147.32) (width 0.4) (layer F.Cu) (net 12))
 (segment (start 127.508 151.384) (end 129.032 149.86) (width 0.4) (layer F.Cu) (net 12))
 (segment (start 168.61 169.93) (end 168.61 174.544) (width 0.4) (layer F.Cu) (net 34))
 (segment (start 168.61 174.544) (end 167.132 176.022) (width 0.4) (layer F.Cu) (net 34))
 (segment (start 148.844 167.64) (end 163.322 167.64) (width 0.4) (layer F.Cu) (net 34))
 (segment (start 165.612 169.93) (end 168.61 169.93) (width 0.4) (layer F.Cu) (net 34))
 (segment (start 163.322 167.64) (end 165.612 169.93) (width 0.4) (layer F.Cu) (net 34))
 (segment (start 168.61 169.93) (end 168.61 164.292) (width 0.4) (layer B.Cu) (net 34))
 (segment (start 165.1 148.336) (end 162.56 145.796) (width 0.4) (layer B.Cu) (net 34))
 (segment (start 165.1 160.782) (end 165.1 148.336) (width 0.4) (layer B.Cu) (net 34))
 (segment (start 168.61 164.292) (end 165.1 160.782) (width 0.4) (layer B.Cu) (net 34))
 (segment (start 149.098 174.244) (end 151.384 174.244) (width 0.5) (layer F.Cu) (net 28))
 (segment (start 119.126 121.158) (end 119.126 128.27) (width 0.5) (layer F.Cu) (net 28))
 (segment (start 117.602 119.634) (end 119.126 121.158) (width 0.5) (layer F.Cu) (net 28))
 (segment (start 111.506 119.634) (end 117.602 119.634) (width 0.5) (layer F.Cu) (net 28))
 (segment (start 105.41 125.73) (end 111.506 119.634) (width 0.5) (layer F.Cu) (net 28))
 (segment (start 105.41 130.81) (end 105.41 125.73) (width 0.5) (layer F.Cu) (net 28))
 (segment (start 100.584 135.636) (end 105.41 130.81) (width 0.5) (layer F.Cu) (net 28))
 (segment (start 100.584 153.924) (end 100.584 135.636) (width 0.5) (layer F.Cu) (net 28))
 (segment (start 106.426 159.766) (end 100.584 153.924) (width 0.5) (layer F.Cu) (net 28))
 (segment (start 121.158 159.766) (end 106.426 159.766) (width 0.5) (layer F.Cu) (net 28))
 (segment (start 122.936 161.544) (end 121.158 159.766) (width 0.5) (layer F.Cu) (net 28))
 (segment (start 122.936 172.974) (end 122.936 161.544) (width 0.5) (layer F.Cu) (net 28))
 (segment (start 128.362002 178.400002) (end 122.936 172.974) (width 0.5) (layer F.Cu) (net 28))
 (segment (start 151.037998 178.400002) (end 128.362002 178.400002) (width 0.5) (layer F.Cu) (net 28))
 (segment (start 151.384 178.054) (end 151.037998 178.400002) (width 0.5) (layer F.Cu) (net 28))
 (segment (start 151.384 174.244) (end 151.384 178.054) (width 0.5) (layer F.Cu) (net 28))
 (segment (start 149.098 176.276) (end 149.098 174.244) (width 0.454) (layer F.Cu) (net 28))
 (segment (start 149.098 174.244) (end 149.098 172.212) (width 0.454) (layer F.Cu) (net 28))
 (segment (start 134.112 151.384) (end 139.446 151.384) (width 0.5) (layer F.Cu) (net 10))
 (segment (start 149.606 137.414) (end 147.066 137.414) (width 0.5) (layer F.Cu) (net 10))
 (segment (start 151.384 139.192) (end 149.606 137.414) (width 0.5) (layer F.Cu) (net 10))
 (segment (start 151.384 144.78) (end 151.384 139.192) (width 0.5) (layer F.Cu) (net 10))
 (segment (start 148.082 148.082) (end 151.384 144.78) (width 0.5) (layer F.Cu) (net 10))
 (segment (start 142.748 148.082) (end 148.082 148.082) (width 0.5) (layer F.Cu) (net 10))
 (segment (start 139.446 151.384) (end 142.748 148.082) (width 0.5) (layer F.Cu) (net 10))
 (segment (start 147.066 137.414) (end 147.066 129.54) (width 0.5) (layer F.Cu) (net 10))
 (segment (start 152.654 129.54) (end 157.734 129.54) (width 0.5) (layer F.Cu) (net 10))
 (segment (start 157.734 129.54) (end 158.496 130.302) (width 0.5) (layer F.Cu) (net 10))
 (segment (start 133.9088 123.4186) (end 133.9088 125.5268) (width 0.5) (layer F.Cu) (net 10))
 (segment (start 153.67 128.524) (end 153.67 124.968) (width 0.5) (layer F.Cu) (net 10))
 (segment (start 152.654 129.54) (end 153.67 128.524) (width 0.5) (layer F.Cu) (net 10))
 (segment (start 137.922 129.54) (end 147.066 129.54) (width 0.5) (layer F.Cu) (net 10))
 (segment (start 147.066 129.54) (end 152.654 129.54) (width 0.5) (layer F.Cu) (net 10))
 (segment (start 133.9088 125.5268) (end 137.922 129.54) (width 0.5) (layer F.Cu) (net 10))
 (segment (start 146.304 114.046) (end 146.304 107.696) (width 0.5) (layer F.Cu) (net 10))
 (segment (start 155.702 98.298) (end 161.036 98.298) (width 0.5) (layer F.Cu) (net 10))
 (segment (start 146.304 107.696) (end 155.702 98.298) (width 0.5) (layer F.Cu) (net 10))
 (segment (start 131.826 114.046) (end 145.034 114.046) (width 0.5) (layer F.Cu) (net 10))
 (segment (start 145.034 114.046) (end 146.304 114.046) (width 0.5) (layer F.Cu) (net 10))
 (segment (start 133.9088 111.2266) (end 133.6294 111.2266) (width 0.5) (layer F.Cu) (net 10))
 (segment (start 131.826 121.3358) (end 133.9088 123.4186) (width 0.5) (layer F.Cu) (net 10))
 (segment (start 131.826 113.03) (end 131.826 114.046) (width 0.5) (layer F.Cu) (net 10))
 (segment (start 131.826 114.046) (end 131.826 121.3358) (width 0.5) (layer F.Cu) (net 10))
 (segment (start 133.6294 111.2266) (end 131.826 113.03) (width 0.5) (layer F.Cu) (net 10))
 (segment (start 125.984 158.496) (end 128.778 158.496) (width 0.5) (layer F.Cu) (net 10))
 (segment (start 134.112 153.162) (end 134.112 151.384) (width 0.5) (layer F.Cu) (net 10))
 (segment (start 134.112 151.384) (end 134.112 147.32) (width 0.5) (layer F.Cu) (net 10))
 (segment (start 128.778 158.496) (end 134.112 153.162) (width 0.5) (layer F.Cu) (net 10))
 (segment (start 122.428 154.432) (end 122.428 156.21) (width 0.5) (layer F.Cu) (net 10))
 (segment (start 124.46 158.242) (end 125.73 158.242) (width 0.5) (layer F.Cu) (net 10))
 (segment (start 122.428 156.21) (end 124.46 158.242) (width 0.5) (layer F.Cu) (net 10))
 (segment (start 141.478 176.276) (end 140.462 176.276) (width 0.5) (layer F.Cu) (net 10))
 (segment (start 125.73 158.242) (end 125.222 158.242) (width 0.5) (layer F.Cu) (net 10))
 (segment (start 125.984 158.496) (end 125.73 158.242) (width 0.5) (layer F.Cu) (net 10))
 (segment (start 125.984 172.974) (end 125.984 158.496) (width 0.5) (layer F.Cu) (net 10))
 (segment (start 130.81 177.546) (end 125.984 172.974) (width 0.5) (layer F.Cu) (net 10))
 (segment (start 138.938 177.546) (end 130.81 177.546) (width 0.5) (layer F.Cu) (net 10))
 (segment (start 140.462 176.276) (end 138.938 177.546) (width 0.5) (layer F.Cu) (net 10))
 (segment (start 136.2075 173.228) (end 140.462 173.228) (width 0.454) (layer F.Cu) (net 3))
 (segment (start 140.462 173.228) (end 141.478 172.212) (width 0.454) (layer F.Cu) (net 3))
 (segment (start 136.2075 175.7045) (end 136.2075 173.228) (width 0.454) (layer F.Cu) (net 3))
 (segment (start 156.51 169.93) (end 157.222 169.93) (width 0.4) (layer B.Cu) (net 1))
 (segment (start 158.75 147.066) (end 160.02 145.796) (width 0.4) (layer B.Cu) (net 1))
 (segment (start 158.75 168.402) (end 158.75 147.066) (width 0.4) (layer B.Cu) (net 1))
 (segment (start 157.222 169.93) (end 158.75 168.402) (width 0.4) (layer B.Cu) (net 1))
 (segment (start 156.51 169.93) (end 156.51 173.02) (width 0.4) (layer F.Cu) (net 1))
 (segment (start 156.51 173.02) (end 159.512 176.022) (width 0.4) (layer F.Cu) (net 1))
 (segment (start 117.1575 165.1) (end 117.1575 162.6235) (width 0.4) (layer F.Cu) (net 7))
 (segment (start 104.59466 169.672) (end 104.59466 168.45534) (width 0.4) (layer F.Cu) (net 7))
 (segment (start 107.95 165.1) (end 117.1575 165.1) (width 0.4) (layer F.Cu) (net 7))
 (segment (start 104.59466 168.45534) (end 107.95 165.1) (width 0.4) (layer F.Cu) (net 7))
 (segment (start 117.1575 173.228) (end 117.1575 175.7045) (width 0.454) (layer F.Cu) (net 6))
 (segment (start 110.59414 169.672) (end 115.57 169.672) (width 0.454) (layer F.Cu) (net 6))
 (segment (start 117.1575 171.2595) (end 117.1575 173.228) (width 0.454) (layer F.Cu) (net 6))
 (segment (start 115.57 169.672) (end 117.1575 171.2595) (width 0.454) (layer F.Cu) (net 6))
 (segment (start 156.51 157.83) (end 159.862 157.83) (width 0.4) (layer F.Cu) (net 31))
 (segment (start 171.196 151.384) (end 171.196 150.114) (width 0.4) (layer F.Cu) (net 31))
 (segment (start 164.592 157.988) (end 171.196 151.384) (width 0.4) (layer F.Cu) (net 31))
 (segment (start 160.02 157.988) (end 164.592 157.988) (width 0.4) (layer F.Cu) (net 31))
 (segment (start 159.862 157.83) (end 160.02 157.988) (width 0.4) (layer F.Cu) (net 31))
 (segment (start 168.61 157.83) (end 168.61 146.004) (width 0.4) (layer B.Cu) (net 29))
 (segment (start 169.58 145.034) (end 171.196 145.034) (width 0.4) (layer B.Cu) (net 29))
 (segment (start 168.61 146.004) (end 169.58 145.034) (width 0.4) (layer B.Cu) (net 29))
 (segment (start 162.56 155.83) (end 162.56 152.146) (width 0.4) (layer F.Cu) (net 30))
 (segment (start 167.132 147.574) (end 171.196 147.574) (width 0.4) (layer F.Cu) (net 30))
 (segment (start 162.56 152.146) (end 167.132 147.574) (width 0.4) (layer F.Cu) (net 30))
 (segment (start 141.224 167.64) (end 141.224 164.592) (width 0.4) (layer F.Cu) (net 8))
 (segment (start 141.224 164.592) (end 141.224 161.544) (width 0.4) (layer F.Cu) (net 8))
 (segment (start 136.144 165.1) (end 140.716 165.1) (width 0.4) (layer F.Cu) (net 8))
 (segment (start 140.716 165.1) (end 141.224 164.592) (width 0.4) (layer F.Cu) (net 8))
 (segment (start 136.2075 162.6235) (end 136.2075 165.0365) (width 0.4) (layer F.Cu) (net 8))
 (segment (start 136.2075 165.0365) (end 136.144 165.1) (width 0.4) (layer F.Cu) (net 8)))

